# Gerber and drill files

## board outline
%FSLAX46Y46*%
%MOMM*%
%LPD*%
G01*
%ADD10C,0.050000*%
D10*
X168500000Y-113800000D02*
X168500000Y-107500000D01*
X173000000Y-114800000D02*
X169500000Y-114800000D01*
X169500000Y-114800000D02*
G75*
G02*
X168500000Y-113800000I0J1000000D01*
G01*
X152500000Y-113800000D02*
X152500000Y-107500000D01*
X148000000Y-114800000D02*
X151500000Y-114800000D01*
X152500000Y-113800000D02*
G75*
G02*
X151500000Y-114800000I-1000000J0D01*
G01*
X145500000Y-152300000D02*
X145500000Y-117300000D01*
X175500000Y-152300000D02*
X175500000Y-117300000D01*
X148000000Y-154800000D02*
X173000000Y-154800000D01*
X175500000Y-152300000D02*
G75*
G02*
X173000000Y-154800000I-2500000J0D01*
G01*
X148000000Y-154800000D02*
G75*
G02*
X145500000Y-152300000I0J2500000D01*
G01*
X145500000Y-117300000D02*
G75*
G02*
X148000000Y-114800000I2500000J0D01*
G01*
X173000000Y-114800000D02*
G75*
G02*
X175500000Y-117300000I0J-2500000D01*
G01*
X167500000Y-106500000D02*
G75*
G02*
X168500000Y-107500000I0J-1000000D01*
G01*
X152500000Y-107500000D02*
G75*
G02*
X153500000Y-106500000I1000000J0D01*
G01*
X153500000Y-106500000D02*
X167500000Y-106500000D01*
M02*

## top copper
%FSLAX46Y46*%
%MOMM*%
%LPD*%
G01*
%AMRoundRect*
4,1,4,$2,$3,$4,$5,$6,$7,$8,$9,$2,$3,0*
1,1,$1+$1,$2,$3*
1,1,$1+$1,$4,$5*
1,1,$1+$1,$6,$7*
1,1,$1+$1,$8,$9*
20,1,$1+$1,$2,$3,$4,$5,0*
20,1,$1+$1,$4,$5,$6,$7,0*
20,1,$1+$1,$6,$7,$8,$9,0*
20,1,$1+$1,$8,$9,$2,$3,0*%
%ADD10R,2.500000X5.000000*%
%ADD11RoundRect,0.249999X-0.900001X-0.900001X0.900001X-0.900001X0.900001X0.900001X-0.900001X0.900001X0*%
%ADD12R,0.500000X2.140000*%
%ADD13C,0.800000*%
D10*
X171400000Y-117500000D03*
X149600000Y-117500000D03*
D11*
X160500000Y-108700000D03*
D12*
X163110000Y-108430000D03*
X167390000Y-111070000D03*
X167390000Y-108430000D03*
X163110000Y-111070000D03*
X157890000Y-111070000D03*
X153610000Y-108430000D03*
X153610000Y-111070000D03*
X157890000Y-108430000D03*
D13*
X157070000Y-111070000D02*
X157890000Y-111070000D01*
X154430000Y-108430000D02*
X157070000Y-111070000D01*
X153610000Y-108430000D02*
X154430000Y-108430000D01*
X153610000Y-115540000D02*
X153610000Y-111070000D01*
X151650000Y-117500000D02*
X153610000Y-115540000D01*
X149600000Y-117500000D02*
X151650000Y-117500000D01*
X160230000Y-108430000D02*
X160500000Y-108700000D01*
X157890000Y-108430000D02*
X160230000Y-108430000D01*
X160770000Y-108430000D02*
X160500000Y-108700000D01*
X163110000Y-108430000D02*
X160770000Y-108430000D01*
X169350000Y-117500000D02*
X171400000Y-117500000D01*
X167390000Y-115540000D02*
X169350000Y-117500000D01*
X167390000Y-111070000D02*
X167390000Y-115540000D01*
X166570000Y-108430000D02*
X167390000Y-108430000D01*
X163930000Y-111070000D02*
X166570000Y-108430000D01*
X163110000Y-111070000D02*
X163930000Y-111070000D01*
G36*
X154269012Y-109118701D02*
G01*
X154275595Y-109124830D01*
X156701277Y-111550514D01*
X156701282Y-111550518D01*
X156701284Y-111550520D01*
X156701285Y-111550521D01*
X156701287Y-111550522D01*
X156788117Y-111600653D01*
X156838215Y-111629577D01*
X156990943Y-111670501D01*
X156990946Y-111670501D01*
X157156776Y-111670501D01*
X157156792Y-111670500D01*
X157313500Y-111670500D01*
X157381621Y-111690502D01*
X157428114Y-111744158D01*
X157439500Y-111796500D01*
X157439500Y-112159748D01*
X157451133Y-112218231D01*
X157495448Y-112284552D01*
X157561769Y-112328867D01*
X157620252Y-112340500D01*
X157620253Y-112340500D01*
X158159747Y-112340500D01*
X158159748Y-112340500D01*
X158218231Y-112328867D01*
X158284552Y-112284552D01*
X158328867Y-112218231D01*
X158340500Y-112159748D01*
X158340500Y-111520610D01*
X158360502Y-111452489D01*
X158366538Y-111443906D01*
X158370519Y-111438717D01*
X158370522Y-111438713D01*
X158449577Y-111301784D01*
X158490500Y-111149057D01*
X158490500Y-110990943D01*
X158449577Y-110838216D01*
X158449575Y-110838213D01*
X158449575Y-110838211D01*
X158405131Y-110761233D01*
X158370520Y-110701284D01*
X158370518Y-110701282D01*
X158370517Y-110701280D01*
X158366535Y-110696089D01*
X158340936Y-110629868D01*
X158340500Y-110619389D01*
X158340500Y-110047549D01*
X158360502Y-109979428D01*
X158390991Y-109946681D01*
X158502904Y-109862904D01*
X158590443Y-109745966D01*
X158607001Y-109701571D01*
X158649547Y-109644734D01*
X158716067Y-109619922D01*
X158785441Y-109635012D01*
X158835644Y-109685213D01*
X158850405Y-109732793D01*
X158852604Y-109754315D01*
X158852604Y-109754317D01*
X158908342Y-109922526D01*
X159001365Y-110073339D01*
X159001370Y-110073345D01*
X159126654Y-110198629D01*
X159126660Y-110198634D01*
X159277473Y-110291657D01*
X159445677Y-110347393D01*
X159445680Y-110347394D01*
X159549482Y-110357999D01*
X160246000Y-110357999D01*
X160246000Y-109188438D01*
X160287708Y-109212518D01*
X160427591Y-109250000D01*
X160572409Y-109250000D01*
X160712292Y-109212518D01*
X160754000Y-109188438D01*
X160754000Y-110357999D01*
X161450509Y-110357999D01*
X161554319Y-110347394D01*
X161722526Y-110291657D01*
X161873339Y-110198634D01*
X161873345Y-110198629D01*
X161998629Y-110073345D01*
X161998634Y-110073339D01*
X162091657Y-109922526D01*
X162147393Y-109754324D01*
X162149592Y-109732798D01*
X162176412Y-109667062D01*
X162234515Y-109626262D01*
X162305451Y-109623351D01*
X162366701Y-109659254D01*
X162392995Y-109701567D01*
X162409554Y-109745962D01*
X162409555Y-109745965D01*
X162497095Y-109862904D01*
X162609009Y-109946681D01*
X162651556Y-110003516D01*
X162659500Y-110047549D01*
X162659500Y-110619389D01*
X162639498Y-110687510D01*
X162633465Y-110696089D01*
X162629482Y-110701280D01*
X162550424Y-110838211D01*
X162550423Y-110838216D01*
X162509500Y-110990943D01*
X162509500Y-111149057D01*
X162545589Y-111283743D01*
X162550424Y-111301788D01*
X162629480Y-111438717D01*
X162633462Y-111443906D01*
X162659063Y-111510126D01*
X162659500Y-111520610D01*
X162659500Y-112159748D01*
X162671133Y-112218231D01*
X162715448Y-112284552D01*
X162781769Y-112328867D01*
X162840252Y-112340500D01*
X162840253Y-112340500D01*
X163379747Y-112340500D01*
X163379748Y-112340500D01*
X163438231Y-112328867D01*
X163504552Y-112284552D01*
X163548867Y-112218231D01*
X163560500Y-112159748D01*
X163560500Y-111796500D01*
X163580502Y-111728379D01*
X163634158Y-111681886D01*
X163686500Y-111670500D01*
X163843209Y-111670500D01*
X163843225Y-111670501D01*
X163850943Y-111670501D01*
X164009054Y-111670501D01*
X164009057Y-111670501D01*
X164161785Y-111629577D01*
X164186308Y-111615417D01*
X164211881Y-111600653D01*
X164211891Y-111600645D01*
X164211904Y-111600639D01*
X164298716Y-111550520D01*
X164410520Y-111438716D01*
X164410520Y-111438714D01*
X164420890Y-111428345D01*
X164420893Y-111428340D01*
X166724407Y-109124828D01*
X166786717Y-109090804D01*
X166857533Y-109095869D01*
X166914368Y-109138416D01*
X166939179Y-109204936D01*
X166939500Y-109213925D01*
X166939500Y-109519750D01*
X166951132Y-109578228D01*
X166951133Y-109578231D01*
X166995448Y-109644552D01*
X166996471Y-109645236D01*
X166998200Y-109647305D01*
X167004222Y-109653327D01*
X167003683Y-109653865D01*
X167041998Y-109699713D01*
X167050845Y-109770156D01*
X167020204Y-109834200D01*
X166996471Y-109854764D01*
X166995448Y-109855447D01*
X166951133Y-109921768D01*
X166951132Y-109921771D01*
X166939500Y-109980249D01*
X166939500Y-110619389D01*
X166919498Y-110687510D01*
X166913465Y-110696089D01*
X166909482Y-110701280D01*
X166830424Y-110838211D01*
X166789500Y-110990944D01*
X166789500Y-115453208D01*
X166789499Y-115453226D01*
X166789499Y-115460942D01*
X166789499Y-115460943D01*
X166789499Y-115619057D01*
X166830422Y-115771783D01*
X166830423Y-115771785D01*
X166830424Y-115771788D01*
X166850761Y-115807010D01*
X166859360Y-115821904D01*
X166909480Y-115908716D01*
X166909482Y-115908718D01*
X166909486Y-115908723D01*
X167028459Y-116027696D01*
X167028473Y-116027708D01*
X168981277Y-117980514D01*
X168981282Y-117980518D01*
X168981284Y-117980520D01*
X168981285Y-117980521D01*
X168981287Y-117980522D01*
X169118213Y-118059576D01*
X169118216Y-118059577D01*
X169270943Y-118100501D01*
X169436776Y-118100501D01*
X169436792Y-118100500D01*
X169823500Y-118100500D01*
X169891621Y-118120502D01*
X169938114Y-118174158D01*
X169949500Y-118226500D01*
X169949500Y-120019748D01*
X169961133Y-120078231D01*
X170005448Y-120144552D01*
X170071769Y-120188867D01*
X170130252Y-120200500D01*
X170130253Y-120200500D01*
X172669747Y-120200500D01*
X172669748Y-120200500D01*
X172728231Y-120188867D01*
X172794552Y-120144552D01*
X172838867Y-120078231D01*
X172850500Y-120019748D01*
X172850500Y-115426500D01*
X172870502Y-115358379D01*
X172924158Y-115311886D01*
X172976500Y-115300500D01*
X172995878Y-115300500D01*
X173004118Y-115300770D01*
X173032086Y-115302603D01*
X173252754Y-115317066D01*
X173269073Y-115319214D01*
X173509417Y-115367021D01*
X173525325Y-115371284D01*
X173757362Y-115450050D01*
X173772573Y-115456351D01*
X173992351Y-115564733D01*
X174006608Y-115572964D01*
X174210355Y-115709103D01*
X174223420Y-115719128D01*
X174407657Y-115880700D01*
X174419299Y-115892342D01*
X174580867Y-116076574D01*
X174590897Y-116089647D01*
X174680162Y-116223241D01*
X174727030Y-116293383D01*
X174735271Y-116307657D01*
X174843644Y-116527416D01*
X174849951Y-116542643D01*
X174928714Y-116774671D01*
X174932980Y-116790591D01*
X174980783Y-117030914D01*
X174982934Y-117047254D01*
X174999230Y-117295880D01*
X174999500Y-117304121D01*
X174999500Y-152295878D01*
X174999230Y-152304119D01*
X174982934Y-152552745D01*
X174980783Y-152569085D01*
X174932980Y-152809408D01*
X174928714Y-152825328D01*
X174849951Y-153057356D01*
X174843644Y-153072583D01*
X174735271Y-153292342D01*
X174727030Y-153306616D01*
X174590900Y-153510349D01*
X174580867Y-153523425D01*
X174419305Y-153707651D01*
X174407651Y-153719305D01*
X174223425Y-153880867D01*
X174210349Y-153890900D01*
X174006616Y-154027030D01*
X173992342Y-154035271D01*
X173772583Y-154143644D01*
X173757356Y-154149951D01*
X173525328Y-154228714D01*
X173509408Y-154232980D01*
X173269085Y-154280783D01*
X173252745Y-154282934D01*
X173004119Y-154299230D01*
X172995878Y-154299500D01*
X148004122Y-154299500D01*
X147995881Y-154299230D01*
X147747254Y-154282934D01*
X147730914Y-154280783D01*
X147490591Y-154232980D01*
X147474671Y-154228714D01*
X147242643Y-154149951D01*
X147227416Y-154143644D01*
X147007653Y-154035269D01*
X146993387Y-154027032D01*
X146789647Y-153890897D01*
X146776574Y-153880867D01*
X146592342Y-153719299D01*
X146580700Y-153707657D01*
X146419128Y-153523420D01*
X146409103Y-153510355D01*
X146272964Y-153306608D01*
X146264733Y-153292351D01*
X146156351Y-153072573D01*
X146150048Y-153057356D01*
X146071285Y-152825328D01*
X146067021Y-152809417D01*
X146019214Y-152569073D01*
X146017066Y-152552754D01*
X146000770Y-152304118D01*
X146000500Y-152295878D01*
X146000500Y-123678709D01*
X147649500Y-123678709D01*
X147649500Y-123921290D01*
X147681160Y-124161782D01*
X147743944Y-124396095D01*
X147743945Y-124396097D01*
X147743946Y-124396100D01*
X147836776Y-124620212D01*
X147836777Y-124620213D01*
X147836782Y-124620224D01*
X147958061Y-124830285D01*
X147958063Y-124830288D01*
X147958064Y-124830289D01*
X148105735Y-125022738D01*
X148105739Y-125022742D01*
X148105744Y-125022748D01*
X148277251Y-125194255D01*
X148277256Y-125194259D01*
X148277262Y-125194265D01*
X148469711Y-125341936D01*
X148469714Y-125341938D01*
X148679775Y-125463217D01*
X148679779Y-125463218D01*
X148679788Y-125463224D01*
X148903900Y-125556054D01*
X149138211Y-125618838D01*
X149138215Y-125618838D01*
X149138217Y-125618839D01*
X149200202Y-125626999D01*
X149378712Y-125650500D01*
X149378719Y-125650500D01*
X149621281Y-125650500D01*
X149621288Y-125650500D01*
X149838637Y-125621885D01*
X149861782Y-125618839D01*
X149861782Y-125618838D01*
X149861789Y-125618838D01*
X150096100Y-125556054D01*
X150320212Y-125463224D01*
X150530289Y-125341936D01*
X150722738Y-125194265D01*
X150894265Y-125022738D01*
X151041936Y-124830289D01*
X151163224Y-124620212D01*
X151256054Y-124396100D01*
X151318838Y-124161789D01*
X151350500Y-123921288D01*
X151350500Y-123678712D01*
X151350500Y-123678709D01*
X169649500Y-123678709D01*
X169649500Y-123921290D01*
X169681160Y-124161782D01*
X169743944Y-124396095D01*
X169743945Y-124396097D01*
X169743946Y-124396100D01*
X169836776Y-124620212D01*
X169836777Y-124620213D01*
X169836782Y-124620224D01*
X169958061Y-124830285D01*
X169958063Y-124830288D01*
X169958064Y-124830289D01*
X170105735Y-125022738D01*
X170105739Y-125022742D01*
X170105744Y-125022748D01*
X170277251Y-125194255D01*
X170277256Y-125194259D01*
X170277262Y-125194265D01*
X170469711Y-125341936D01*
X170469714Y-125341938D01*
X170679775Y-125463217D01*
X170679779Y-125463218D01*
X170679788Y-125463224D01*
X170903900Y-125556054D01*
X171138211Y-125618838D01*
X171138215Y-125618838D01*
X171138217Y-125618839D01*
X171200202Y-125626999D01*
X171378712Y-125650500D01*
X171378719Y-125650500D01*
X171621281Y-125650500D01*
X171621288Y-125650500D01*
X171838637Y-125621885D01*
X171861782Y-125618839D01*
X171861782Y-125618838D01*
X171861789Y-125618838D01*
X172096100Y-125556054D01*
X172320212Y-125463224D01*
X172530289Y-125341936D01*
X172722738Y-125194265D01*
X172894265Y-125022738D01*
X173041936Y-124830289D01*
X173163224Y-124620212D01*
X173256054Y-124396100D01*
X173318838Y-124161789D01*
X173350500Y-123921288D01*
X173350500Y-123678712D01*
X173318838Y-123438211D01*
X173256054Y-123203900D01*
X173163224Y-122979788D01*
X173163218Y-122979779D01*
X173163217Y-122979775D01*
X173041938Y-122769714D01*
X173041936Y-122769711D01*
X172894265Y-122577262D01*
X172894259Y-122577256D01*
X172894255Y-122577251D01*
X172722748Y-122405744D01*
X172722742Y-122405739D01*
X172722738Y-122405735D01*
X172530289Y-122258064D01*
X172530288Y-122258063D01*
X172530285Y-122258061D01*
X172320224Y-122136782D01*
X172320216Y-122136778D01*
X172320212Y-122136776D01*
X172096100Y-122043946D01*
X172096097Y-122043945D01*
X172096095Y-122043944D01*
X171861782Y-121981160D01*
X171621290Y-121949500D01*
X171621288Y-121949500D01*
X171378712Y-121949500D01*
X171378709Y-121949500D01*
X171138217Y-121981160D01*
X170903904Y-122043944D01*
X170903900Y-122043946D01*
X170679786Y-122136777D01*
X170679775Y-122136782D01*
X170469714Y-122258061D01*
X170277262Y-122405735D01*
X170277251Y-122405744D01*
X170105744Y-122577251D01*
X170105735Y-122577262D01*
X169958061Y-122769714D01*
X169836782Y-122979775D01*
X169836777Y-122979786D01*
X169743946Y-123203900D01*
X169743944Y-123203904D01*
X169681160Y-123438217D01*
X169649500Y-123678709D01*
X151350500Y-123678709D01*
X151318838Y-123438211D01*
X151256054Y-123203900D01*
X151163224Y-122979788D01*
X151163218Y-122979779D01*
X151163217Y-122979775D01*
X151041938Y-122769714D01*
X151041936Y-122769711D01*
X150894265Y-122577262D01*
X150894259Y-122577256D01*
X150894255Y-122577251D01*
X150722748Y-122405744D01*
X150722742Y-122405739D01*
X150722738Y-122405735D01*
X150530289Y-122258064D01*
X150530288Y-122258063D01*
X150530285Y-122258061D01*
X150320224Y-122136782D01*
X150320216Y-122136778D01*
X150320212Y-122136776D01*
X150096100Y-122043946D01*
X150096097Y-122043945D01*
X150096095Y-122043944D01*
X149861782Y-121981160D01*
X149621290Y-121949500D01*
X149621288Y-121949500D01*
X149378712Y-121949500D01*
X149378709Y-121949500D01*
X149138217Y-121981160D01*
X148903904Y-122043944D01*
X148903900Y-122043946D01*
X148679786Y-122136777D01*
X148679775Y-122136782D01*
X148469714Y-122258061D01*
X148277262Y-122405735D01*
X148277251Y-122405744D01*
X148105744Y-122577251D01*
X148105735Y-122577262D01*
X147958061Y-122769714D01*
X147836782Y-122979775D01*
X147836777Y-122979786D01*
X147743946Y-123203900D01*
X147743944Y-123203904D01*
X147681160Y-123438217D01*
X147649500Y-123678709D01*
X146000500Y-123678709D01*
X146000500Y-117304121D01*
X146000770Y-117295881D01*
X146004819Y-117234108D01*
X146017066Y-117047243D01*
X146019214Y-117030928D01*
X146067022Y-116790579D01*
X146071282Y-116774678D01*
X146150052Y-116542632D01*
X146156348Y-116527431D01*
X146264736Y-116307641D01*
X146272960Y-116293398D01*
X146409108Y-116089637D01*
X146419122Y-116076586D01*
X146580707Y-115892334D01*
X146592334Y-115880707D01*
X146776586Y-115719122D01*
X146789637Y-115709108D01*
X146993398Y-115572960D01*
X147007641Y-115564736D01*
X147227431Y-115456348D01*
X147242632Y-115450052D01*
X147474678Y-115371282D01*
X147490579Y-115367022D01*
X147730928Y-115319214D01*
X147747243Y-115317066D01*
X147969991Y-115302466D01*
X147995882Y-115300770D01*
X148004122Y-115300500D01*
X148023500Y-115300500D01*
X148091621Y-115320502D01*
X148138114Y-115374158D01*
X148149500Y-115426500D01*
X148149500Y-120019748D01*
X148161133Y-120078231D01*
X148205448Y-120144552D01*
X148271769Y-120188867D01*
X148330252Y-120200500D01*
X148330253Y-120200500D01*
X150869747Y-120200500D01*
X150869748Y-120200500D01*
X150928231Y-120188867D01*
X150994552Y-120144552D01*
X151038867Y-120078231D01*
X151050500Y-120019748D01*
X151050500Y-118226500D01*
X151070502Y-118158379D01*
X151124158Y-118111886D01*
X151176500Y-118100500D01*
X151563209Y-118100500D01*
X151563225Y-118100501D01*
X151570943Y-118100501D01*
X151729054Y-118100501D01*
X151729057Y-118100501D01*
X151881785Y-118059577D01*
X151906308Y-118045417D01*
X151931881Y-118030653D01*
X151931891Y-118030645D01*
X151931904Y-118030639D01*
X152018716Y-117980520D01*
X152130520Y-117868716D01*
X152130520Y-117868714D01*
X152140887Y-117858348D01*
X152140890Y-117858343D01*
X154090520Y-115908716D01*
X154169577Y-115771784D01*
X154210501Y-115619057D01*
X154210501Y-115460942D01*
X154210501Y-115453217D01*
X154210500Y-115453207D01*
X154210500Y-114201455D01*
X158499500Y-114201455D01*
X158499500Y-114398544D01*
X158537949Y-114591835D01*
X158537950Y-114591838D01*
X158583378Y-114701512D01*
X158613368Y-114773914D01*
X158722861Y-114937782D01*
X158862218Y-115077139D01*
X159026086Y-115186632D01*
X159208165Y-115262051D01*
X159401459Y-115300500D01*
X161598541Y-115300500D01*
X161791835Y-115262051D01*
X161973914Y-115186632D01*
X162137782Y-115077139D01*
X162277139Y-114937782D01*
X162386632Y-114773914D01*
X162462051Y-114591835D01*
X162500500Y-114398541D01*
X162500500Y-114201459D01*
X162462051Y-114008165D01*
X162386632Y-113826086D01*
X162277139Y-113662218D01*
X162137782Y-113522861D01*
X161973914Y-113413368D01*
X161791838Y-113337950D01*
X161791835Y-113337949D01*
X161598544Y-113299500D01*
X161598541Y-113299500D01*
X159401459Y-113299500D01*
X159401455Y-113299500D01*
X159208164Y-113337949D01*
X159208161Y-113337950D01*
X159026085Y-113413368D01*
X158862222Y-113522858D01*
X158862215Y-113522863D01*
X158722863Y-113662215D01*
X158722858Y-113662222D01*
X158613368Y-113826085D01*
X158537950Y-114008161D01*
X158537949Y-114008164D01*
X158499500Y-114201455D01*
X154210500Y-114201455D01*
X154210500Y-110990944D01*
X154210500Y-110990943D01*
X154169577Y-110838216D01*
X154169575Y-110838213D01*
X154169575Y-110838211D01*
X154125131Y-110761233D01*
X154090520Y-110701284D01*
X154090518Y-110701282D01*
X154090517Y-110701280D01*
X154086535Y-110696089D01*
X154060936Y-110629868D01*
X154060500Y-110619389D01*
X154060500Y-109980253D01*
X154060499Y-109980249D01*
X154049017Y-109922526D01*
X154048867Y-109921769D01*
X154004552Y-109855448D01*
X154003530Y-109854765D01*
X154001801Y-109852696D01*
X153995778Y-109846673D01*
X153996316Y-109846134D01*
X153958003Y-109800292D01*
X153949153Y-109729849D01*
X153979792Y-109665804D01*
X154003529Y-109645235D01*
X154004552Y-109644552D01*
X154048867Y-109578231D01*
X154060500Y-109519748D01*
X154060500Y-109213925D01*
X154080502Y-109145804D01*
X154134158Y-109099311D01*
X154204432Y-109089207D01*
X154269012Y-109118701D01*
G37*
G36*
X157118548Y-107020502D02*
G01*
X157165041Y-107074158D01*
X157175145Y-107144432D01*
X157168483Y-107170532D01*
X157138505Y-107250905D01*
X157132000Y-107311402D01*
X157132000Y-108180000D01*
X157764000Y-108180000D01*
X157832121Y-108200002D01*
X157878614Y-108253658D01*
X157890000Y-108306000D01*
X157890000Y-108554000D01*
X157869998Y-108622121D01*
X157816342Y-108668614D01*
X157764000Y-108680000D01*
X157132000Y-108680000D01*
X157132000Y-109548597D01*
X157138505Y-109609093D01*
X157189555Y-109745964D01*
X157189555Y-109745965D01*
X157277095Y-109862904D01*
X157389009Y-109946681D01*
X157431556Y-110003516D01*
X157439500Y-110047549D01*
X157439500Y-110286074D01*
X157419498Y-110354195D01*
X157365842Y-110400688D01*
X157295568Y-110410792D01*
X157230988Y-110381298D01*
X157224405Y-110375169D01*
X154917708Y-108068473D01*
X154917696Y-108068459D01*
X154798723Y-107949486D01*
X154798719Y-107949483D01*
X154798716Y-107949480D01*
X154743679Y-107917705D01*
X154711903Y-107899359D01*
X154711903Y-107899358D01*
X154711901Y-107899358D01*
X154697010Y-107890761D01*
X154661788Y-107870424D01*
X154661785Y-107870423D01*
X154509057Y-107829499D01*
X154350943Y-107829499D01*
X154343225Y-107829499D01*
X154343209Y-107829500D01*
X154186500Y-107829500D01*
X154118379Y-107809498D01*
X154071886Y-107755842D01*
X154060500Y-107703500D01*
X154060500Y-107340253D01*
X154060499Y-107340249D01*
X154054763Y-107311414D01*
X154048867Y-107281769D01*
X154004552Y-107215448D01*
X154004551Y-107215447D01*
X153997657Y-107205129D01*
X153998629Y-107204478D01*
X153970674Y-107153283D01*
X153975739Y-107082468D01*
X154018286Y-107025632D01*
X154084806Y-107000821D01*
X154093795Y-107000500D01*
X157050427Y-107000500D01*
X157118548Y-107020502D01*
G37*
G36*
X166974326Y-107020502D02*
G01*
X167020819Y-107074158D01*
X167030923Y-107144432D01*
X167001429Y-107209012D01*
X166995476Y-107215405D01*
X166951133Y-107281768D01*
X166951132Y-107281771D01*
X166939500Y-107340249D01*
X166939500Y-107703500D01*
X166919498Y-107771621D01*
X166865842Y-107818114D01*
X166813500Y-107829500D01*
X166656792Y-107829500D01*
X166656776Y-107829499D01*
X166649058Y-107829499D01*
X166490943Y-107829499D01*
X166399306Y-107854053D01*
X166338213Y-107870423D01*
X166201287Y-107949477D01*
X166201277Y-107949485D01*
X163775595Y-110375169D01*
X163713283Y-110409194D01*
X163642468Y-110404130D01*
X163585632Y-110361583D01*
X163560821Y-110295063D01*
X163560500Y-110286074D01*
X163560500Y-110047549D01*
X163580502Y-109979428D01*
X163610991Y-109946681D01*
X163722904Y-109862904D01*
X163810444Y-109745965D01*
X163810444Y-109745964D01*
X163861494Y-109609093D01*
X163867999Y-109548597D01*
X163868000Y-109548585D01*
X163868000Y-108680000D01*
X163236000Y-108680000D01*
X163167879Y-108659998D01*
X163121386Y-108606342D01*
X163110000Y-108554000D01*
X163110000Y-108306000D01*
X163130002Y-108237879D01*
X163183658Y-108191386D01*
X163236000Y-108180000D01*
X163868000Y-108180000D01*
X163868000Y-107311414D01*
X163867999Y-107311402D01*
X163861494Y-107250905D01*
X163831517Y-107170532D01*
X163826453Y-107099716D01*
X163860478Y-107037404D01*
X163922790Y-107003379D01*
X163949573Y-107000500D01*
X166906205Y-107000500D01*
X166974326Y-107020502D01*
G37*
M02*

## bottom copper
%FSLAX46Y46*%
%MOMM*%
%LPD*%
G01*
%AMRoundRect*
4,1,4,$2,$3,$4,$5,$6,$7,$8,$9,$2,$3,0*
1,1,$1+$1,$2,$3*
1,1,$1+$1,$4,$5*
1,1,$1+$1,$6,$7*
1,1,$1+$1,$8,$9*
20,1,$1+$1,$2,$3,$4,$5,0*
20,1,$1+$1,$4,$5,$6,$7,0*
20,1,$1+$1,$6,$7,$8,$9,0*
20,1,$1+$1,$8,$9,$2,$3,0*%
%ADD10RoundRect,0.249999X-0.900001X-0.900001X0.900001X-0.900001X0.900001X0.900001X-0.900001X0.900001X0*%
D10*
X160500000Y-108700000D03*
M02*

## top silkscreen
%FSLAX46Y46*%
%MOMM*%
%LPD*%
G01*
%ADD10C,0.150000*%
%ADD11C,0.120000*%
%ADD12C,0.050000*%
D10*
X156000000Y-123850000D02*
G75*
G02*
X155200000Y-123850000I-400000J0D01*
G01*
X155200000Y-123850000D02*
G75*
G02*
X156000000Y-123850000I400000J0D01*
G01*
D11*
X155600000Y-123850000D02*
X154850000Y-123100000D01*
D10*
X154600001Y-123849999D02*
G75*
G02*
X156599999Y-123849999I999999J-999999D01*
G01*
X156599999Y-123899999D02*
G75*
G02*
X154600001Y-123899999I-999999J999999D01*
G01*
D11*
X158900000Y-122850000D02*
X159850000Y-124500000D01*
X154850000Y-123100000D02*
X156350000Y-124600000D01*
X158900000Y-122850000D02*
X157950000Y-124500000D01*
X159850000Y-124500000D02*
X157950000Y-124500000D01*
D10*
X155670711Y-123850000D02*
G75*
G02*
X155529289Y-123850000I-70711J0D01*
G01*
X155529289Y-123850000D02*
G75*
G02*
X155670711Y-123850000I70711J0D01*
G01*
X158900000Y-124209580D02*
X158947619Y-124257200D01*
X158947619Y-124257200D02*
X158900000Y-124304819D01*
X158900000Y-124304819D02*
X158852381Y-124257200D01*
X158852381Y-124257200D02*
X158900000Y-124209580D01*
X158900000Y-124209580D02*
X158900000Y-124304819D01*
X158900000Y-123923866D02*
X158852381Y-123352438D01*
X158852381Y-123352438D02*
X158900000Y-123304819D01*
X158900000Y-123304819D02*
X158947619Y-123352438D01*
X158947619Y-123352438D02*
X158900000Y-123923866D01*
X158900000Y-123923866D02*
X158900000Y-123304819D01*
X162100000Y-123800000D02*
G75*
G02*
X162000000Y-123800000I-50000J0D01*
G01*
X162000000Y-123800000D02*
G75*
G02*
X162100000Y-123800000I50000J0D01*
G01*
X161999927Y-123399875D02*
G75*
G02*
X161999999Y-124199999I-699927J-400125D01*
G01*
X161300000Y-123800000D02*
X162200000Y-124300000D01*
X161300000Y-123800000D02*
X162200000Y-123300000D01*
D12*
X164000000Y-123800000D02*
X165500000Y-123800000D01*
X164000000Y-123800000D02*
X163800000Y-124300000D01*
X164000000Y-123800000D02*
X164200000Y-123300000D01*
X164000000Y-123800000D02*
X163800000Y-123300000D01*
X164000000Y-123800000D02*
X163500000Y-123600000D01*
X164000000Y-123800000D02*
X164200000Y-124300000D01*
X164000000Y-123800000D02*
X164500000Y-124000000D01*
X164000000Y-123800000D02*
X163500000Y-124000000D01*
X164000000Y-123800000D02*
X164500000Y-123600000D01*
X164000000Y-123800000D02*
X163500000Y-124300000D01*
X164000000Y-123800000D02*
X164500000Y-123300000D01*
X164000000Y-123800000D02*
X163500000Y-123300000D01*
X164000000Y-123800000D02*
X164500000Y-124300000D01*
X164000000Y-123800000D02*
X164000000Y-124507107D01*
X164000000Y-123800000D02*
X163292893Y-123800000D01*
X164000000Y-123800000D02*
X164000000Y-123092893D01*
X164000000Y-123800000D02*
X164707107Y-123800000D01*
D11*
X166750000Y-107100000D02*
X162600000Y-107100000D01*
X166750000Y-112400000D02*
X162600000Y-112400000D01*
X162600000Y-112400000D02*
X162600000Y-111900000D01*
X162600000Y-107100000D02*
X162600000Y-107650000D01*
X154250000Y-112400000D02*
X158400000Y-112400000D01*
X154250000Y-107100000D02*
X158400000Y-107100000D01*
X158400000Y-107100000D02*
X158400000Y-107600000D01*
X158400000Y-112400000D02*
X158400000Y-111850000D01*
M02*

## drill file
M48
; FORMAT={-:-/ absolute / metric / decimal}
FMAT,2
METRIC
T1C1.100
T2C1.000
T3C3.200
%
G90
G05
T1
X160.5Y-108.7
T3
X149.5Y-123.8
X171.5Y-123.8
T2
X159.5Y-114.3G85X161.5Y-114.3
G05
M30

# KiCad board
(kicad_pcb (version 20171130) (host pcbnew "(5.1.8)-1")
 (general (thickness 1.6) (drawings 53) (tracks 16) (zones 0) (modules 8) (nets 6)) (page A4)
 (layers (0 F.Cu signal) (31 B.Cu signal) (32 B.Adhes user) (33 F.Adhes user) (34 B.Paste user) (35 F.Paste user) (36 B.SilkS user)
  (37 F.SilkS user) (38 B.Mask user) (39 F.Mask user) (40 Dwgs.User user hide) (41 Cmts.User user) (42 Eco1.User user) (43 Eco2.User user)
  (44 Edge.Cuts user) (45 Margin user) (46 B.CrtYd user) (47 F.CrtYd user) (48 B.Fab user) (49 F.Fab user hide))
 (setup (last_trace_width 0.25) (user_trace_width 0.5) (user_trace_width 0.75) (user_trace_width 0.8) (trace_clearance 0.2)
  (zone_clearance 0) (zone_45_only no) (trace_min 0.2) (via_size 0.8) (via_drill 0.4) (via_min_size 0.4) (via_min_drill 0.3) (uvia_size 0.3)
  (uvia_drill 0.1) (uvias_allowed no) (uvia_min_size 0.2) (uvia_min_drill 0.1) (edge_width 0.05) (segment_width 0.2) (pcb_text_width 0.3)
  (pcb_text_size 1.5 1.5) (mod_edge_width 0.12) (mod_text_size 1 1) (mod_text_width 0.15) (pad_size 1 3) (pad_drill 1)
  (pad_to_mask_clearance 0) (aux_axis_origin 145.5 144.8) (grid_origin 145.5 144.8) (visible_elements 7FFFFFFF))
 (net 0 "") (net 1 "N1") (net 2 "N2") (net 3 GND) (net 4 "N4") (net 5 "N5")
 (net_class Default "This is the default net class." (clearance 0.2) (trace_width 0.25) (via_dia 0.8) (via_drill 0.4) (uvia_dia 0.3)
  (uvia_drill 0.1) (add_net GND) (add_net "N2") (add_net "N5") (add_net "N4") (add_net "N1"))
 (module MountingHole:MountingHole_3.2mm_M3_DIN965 (layer F.Cu) (at 171.5 123.8)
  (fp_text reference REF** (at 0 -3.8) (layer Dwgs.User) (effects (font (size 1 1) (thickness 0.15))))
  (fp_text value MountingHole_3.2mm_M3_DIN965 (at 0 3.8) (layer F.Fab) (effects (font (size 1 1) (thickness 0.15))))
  (pad 1 np_thru_hole circle (at 0 0) (size 3.2 3.2) (drill 3.2) (layers *.Cu *.Mask)))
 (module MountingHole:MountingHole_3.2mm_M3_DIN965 (layer F.Cu) (at 149.5 123.8)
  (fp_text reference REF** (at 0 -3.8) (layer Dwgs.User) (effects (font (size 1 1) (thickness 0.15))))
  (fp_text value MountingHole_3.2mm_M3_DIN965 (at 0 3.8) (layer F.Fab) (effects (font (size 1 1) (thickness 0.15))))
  (pad 1 np_thru_hole circle (at 0 0) (size 3.2 3.2) (drill 3.2) (layers *.Cu *.Mask)))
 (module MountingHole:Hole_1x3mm (layer F.Cu) (at 160.5 114.3 90)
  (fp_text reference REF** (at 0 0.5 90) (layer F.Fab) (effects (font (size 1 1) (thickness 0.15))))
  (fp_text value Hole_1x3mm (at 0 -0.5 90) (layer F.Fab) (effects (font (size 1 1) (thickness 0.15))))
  (pad "" np_thru_hole oval (at 0 0 90) (size 1 3) (drill oval 1 3) (layers *.Cu *.Mask)))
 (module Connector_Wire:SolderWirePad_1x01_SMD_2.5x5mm (layer F.Cu) (at 171.4 117.5)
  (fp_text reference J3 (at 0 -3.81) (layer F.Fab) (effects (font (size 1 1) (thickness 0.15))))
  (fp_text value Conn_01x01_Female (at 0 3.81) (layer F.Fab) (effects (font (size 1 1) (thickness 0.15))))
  (pad 1 smd rect (at 0 0) (size 2.5 5) (layers F.Cu F.Paste F.Mask) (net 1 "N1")))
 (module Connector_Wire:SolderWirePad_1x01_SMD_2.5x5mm (layer F.Cu) (at 149.6 117.5)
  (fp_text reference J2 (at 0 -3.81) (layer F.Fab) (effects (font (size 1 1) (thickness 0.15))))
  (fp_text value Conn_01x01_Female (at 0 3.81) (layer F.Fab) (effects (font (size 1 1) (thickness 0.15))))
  (pad 1 smd rect (at 0 0) (size 2.5 5) (layers F.Cu F.Paste F.Mask) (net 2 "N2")))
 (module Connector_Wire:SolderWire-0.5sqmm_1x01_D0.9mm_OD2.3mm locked (layer F.Cu) (at 160.5 108.7)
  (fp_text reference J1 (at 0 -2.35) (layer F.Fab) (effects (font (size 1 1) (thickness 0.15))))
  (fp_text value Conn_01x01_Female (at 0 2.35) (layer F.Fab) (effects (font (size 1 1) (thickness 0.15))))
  (pad 1 thru_hole roundrect (at 0 0) (size 2.3 2.3) (drill 1.1) (layers *.Cu *.Mask) (roundrect_rratio 0.1086952173913043) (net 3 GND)))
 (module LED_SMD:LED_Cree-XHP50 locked (layer F.Cu) (at 165.25 109.75)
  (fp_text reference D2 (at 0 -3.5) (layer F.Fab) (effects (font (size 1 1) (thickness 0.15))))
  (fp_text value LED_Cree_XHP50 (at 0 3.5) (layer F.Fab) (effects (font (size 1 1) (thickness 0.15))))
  (fp_line (start 1.5 -2.65) (end -2.65 -2.65) (layer F.SilkS) (width 0.12))
  (fp_line (start 1.5 2.65) (end -2.65 2.65) (layer F.SilkS) (width 0.12))
  (fp_line (start -2.65 2.65) (end -2.65 2.15) (layer F.SilkS) (width 0.12))
  (fp_line (start -2.65 -2.65) (end -2.65 -2.1) (layer F.SilkS) (width 0.12))
  (pad 2 smd rect (at -2.14 -1.32) (size 0.5 2.14) (layers F.Cu F.Paste F.Mask) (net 3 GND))
  (pad 3 smd rect (at 2.14 1.32) (size 0.5 2.14) (layers F.Cu F.Paste F.Mask) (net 1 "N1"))
  (pad 5 smd rect (at 0 0) (size 2.78 4.78) (layers F.Paste) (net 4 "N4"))
  (pad 1 smd rect (at 2.14 -1.32) (size 0.5 2.14) (layers F.Cu F.Paste F.Mask) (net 4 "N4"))
  (pad 4 smd rect (at -2.14 1.32) (size 0.5 2.14) (layers F.Cu F.Paste F.Mask) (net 4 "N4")))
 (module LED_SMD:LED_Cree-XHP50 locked (layer F.Cu) (at 155.75 109.75 180)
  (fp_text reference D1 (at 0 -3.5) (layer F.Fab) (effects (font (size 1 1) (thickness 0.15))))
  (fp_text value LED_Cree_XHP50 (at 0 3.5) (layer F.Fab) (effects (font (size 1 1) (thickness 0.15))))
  (fp_line (start 1.5 -2.65) (end -2.65 -2.65) (layer F.SilkS) (width 0.12))
  (fp_line (start 1.5 2.65) (end -2.65 2.65) (layer F.SilkS) (width 0.12))
  (fp_line (start -2.65 2.65) (end -2.65 2.15) (layer F.SilkS) (width 0.12))
  (fp_line (start -2.65 -2.65) (end -2.65 -2.1) (layer F.SilkS) (width 0.12))
  (pad 2 smd rect (at -2.14 -1.32 180) (size 0.5 2.14) (layers F.Cu F.Paste F.Mask) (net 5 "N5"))
  (pad 3 smd rect (at 2.14 1.32 180) (size 0.5 2.14) (layers F.Cu F.Paste F.Mask) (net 5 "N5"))
  (pad 5 smd rect (at 0 0 180) (size 2.78 4.78) (layers F.Paste) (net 5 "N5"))
  (pad 1 smd rect (at 2.14 -1.32 180) (size 0.5 2.14) (layers F.Cu F.Paste F.Mask) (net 2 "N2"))
  (pad 4 smd rect (at -2.14 1.32 180) (size 0.5 2.14) (layers F.Cu F.Paste F.Mask) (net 3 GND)))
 (gr_circle (center 155.6 123.85) (end 156 123.85) (layer F.SilkS) (width 0.15))
 (gr_line (start 155.6 123.85) (end 154.85 123.1) (layer F.SilkS) (width 0.12))
 (gr_arc (start 155.6 124.849998) (end 156.599999 123.849999) (angle -90) (layer F.SilkS) (width 0.15))
 (gr_arc (start 155.6 122.9) (end 154.600001 123.899999) (angle -90) (layer F.SilkS) (width 0.15))
 (gr_line (start 158.9 122.85) (end 159.85 124.5) (layer F.SilkS) (width 0.12))
 (gr_line (start 154.85 123.1) (end 156.35 124.6) (layer F.SilkS) (width 0.12))
 (gr_line (start 158.9 122.85) (end 157.95 124.5) (layer F.SilkS) (width 0.12))
 (gr_line (start 159.85 124.5) (end 157.95 124.5) (layer F.SilkS) (width 0.12))
 (gr_circle (center 155.6 123.85) (end 155.670711 123.85) (layer F.SilkS) (width 0.15))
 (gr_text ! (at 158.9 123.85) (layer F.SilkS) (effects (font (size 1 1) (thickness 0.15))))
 (gr_line (start 168.5 113.8) (end 168.5 107.5) (layer Edge.Cuts) (width 0.05))
 (gr_line (start 173 114.8) (end 169.5 114.8) (layer Edge.Cuts) (width 0.05))
 (gr_arc (start 169.5 113.8) (end 168.5 113.8) (angle -90) (layer Edge.Cuts) (width 0.05))
 (gr_line (start 152.5 113.8) (end 152.5 107.5) (layer Edge.Cuts) (width 0.05))
 (gr_line (start 148 114.8) (end 151.5 114.8) (layer Edge.Cuts) (width 0.05))
 (gr_arc (start 151.5 113.8) (end 151.5 114.8) (angle -90) (layer Edge.Cuts) (width 0.05))
 (gr_line (start 145.5 152.3) (end 145.5 117.3) (layer Edge.Cuts) (width 0.05))
 (gr_line (start 175.5 152.3) (end 175.5 117.3) (layer Edge.Cuts) (width 0.05))
 (gr_line (start 148 154.8) (end 173 154.8) (layer Edge.Cuts) (width 0.05))
 (gr_arc (start 173 152.3) (end 173 154.8) (angle -90) (layer Edge.Cuts) (width 0.05))
 (gr_arc (start 148 152.3) (end 145.5 152.3) (angle -90) (layer Edge.Cuts) (width 0.05))
 (gr_arc (start 148 117.3) (end 148 114.8) (angle -90) (layer Edge.Cuts) (width 0.05))
 (gr_arc (start 173 117.3) (end 175.5 117.3) (angle -90) (layer Edge.Cuts) (width 0.05))
 (gr_arc (start 167.5 107.5) (end 168.5 107.5) (angle -90) (layer Edge.Cuts) (width 0.05))
 (gr_arc (start 153.5 107.5) (end 153.5 106.5) (angle -90) (layer Edge.Cuts) (width 0.05))
 (gr_line (start 153.5 106.5) (end 167.5 106.5) (layer Edge.Cuts) (width 0.05))
 (gr_circle (center 162.05 123.8) (end 162.1 123.8) (layer F.SilkS) (width 0.15))
 (gr_arc (start 161.3 123.8) (end 161.999999 124.199999) (angle -59.5) (layer F.SilkS) (width 0.15))
 (gr_line (start 161.3 123.8) (end 162.2 124.3) (layer F.SilkS) (width 0.15))
 (gr_line (start 161.3 123.8) (end 162.2 123.3) (layer F.SilkS) (width 0.15))
 (gr_line (start 164 123.8) (end 165.5 123.8) (layer F.SilkS) (width 0.05))
 (gr_line (start 164 123.8) (end 163.8 124.3) (layer F.SilkS) (width 0.05))
 (gr_line (start 164 123.8) (end 164.2 123.3) (layer F.SilkS) (width 0.05))
 (gr_line (start 164 123.8) (end 163.8 123.3) (layer F.SilkS) (width 0.05))
 (gr_line (start 164 123.8) (end 163.5 123.6) (layer F.SilkS) (width 0.05))
 (gr_line (start 164 123.8) (end 164.2 124.3) (layer F.SilkS) (width 0.05))
 (gr_line (start 164 123.8) (end 164.5 124) (layer F.SilkS) (width 0.05))
 (gr_line (start 164 123.8) (end 163.5 124) (layer F.SilkS) (width 0.05))
 (gr_line (start 164 123.8) (end 164.5 123.6) (layer F.SilkS) (width 0.05))
 (gr_line (start 164 123.8) (end 163.5 124.3) (layer F.SilkS) (width 0.05))
 (gr_line (start 164 123.8) (end 164.5 123.3) (layer F.SilkS) (width 0.05))
 (gr_line (start 164 123.8) (end 163.5 123.3) (layer F.SilkS) (width 0.05))
 (gr_line (start 164 123.8) (end 164.5 124.3) (layer F.SilkS) (width 0.05))
 (gr_line (start 164 123.8) (end 164 124.507107) (layer F.SilkS) (width 0.05))
 (gr_line (start 164 123.8) (end 163.292893 123.8) (layer F.SilkS) (width 0.05))
 (gr_line (start 164 123.8) (end 164 123.092893) (layer F.SilkS) (width 0.05))
 (gr_line (start 164 123.8) (end 164.707107 123.8) (layer F.SilkS) (width 0.05))
 (segment (start 157.07 111.07) (end 157.89 111.07) (width 0.8) (layer F.Cu) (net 5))
 (segment (start 154.43 108.43) (end 157.07 111.07) (width 0.8) (layer F.Cu) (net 5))
 (segment (start 153.61 108.43) (end 154.43 108.43) (width 0.8) (layer F.Cu) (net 5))
 (segment (start 153.61 115.54) (end 153.61 111.07) (width 0.8) (layer F.Cu) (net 2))
 (segment (start 151.65 117.5) (end 153.61 115.54) (width 0.8) (layer F.Cu) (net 2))
 (segment (start 149.6 117.5) (end 151.65 117.5) (width 0.8) (layer F.Cu) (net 2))
 (segment (start 160.23 108.43) (end 160.5 108.7) (width 0.8) (layer F.Cu) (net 3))
 (segment (start 157.89 108.43) (end 160.23 108.43) (width 0.8) (layer F.Cu) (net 3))
 (segment (start 160.77 108.43) (end 160.5 108.7) (width 0.8) (layer F.Cu) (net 3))
 (segment (start 163.11 108.43) (end 160.77 108.43) (width 0.8) (layer F.Cu) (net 3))
 (segment (start 169.35 117.5) (end 171.4 117.5) (width 0.8) (layer F.Cu) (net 1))
 (segment (start 167.39 115.54) (end 169.35 117.5) (width 0.8) (layer F.Cu) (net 1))
 (segment (start 167.39 111.07) (end 167.39 115.54) (width 0.8) (layer F.Cu) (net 1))
 (segment (start 166.57 108.43) (end 167.39 108.43) (width 0.8) (layer F.Cu) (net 4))
 (segment (start 163.93 111.07) (end 166.57 108.43) (width 0.8) (layer F.Cu) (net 4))
 (segment (start 163.11 111.07) (end 163.93 111.07) (width 0.8) (layer F.Cu) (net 4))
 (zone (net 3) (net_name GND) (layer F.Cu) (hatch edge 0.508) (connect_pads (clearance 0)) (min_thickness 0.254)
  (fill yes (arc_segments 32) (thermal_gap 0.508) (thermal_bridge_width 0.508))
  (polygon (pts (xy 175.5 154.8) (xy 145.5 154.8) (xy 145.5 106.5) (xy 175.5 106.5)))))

